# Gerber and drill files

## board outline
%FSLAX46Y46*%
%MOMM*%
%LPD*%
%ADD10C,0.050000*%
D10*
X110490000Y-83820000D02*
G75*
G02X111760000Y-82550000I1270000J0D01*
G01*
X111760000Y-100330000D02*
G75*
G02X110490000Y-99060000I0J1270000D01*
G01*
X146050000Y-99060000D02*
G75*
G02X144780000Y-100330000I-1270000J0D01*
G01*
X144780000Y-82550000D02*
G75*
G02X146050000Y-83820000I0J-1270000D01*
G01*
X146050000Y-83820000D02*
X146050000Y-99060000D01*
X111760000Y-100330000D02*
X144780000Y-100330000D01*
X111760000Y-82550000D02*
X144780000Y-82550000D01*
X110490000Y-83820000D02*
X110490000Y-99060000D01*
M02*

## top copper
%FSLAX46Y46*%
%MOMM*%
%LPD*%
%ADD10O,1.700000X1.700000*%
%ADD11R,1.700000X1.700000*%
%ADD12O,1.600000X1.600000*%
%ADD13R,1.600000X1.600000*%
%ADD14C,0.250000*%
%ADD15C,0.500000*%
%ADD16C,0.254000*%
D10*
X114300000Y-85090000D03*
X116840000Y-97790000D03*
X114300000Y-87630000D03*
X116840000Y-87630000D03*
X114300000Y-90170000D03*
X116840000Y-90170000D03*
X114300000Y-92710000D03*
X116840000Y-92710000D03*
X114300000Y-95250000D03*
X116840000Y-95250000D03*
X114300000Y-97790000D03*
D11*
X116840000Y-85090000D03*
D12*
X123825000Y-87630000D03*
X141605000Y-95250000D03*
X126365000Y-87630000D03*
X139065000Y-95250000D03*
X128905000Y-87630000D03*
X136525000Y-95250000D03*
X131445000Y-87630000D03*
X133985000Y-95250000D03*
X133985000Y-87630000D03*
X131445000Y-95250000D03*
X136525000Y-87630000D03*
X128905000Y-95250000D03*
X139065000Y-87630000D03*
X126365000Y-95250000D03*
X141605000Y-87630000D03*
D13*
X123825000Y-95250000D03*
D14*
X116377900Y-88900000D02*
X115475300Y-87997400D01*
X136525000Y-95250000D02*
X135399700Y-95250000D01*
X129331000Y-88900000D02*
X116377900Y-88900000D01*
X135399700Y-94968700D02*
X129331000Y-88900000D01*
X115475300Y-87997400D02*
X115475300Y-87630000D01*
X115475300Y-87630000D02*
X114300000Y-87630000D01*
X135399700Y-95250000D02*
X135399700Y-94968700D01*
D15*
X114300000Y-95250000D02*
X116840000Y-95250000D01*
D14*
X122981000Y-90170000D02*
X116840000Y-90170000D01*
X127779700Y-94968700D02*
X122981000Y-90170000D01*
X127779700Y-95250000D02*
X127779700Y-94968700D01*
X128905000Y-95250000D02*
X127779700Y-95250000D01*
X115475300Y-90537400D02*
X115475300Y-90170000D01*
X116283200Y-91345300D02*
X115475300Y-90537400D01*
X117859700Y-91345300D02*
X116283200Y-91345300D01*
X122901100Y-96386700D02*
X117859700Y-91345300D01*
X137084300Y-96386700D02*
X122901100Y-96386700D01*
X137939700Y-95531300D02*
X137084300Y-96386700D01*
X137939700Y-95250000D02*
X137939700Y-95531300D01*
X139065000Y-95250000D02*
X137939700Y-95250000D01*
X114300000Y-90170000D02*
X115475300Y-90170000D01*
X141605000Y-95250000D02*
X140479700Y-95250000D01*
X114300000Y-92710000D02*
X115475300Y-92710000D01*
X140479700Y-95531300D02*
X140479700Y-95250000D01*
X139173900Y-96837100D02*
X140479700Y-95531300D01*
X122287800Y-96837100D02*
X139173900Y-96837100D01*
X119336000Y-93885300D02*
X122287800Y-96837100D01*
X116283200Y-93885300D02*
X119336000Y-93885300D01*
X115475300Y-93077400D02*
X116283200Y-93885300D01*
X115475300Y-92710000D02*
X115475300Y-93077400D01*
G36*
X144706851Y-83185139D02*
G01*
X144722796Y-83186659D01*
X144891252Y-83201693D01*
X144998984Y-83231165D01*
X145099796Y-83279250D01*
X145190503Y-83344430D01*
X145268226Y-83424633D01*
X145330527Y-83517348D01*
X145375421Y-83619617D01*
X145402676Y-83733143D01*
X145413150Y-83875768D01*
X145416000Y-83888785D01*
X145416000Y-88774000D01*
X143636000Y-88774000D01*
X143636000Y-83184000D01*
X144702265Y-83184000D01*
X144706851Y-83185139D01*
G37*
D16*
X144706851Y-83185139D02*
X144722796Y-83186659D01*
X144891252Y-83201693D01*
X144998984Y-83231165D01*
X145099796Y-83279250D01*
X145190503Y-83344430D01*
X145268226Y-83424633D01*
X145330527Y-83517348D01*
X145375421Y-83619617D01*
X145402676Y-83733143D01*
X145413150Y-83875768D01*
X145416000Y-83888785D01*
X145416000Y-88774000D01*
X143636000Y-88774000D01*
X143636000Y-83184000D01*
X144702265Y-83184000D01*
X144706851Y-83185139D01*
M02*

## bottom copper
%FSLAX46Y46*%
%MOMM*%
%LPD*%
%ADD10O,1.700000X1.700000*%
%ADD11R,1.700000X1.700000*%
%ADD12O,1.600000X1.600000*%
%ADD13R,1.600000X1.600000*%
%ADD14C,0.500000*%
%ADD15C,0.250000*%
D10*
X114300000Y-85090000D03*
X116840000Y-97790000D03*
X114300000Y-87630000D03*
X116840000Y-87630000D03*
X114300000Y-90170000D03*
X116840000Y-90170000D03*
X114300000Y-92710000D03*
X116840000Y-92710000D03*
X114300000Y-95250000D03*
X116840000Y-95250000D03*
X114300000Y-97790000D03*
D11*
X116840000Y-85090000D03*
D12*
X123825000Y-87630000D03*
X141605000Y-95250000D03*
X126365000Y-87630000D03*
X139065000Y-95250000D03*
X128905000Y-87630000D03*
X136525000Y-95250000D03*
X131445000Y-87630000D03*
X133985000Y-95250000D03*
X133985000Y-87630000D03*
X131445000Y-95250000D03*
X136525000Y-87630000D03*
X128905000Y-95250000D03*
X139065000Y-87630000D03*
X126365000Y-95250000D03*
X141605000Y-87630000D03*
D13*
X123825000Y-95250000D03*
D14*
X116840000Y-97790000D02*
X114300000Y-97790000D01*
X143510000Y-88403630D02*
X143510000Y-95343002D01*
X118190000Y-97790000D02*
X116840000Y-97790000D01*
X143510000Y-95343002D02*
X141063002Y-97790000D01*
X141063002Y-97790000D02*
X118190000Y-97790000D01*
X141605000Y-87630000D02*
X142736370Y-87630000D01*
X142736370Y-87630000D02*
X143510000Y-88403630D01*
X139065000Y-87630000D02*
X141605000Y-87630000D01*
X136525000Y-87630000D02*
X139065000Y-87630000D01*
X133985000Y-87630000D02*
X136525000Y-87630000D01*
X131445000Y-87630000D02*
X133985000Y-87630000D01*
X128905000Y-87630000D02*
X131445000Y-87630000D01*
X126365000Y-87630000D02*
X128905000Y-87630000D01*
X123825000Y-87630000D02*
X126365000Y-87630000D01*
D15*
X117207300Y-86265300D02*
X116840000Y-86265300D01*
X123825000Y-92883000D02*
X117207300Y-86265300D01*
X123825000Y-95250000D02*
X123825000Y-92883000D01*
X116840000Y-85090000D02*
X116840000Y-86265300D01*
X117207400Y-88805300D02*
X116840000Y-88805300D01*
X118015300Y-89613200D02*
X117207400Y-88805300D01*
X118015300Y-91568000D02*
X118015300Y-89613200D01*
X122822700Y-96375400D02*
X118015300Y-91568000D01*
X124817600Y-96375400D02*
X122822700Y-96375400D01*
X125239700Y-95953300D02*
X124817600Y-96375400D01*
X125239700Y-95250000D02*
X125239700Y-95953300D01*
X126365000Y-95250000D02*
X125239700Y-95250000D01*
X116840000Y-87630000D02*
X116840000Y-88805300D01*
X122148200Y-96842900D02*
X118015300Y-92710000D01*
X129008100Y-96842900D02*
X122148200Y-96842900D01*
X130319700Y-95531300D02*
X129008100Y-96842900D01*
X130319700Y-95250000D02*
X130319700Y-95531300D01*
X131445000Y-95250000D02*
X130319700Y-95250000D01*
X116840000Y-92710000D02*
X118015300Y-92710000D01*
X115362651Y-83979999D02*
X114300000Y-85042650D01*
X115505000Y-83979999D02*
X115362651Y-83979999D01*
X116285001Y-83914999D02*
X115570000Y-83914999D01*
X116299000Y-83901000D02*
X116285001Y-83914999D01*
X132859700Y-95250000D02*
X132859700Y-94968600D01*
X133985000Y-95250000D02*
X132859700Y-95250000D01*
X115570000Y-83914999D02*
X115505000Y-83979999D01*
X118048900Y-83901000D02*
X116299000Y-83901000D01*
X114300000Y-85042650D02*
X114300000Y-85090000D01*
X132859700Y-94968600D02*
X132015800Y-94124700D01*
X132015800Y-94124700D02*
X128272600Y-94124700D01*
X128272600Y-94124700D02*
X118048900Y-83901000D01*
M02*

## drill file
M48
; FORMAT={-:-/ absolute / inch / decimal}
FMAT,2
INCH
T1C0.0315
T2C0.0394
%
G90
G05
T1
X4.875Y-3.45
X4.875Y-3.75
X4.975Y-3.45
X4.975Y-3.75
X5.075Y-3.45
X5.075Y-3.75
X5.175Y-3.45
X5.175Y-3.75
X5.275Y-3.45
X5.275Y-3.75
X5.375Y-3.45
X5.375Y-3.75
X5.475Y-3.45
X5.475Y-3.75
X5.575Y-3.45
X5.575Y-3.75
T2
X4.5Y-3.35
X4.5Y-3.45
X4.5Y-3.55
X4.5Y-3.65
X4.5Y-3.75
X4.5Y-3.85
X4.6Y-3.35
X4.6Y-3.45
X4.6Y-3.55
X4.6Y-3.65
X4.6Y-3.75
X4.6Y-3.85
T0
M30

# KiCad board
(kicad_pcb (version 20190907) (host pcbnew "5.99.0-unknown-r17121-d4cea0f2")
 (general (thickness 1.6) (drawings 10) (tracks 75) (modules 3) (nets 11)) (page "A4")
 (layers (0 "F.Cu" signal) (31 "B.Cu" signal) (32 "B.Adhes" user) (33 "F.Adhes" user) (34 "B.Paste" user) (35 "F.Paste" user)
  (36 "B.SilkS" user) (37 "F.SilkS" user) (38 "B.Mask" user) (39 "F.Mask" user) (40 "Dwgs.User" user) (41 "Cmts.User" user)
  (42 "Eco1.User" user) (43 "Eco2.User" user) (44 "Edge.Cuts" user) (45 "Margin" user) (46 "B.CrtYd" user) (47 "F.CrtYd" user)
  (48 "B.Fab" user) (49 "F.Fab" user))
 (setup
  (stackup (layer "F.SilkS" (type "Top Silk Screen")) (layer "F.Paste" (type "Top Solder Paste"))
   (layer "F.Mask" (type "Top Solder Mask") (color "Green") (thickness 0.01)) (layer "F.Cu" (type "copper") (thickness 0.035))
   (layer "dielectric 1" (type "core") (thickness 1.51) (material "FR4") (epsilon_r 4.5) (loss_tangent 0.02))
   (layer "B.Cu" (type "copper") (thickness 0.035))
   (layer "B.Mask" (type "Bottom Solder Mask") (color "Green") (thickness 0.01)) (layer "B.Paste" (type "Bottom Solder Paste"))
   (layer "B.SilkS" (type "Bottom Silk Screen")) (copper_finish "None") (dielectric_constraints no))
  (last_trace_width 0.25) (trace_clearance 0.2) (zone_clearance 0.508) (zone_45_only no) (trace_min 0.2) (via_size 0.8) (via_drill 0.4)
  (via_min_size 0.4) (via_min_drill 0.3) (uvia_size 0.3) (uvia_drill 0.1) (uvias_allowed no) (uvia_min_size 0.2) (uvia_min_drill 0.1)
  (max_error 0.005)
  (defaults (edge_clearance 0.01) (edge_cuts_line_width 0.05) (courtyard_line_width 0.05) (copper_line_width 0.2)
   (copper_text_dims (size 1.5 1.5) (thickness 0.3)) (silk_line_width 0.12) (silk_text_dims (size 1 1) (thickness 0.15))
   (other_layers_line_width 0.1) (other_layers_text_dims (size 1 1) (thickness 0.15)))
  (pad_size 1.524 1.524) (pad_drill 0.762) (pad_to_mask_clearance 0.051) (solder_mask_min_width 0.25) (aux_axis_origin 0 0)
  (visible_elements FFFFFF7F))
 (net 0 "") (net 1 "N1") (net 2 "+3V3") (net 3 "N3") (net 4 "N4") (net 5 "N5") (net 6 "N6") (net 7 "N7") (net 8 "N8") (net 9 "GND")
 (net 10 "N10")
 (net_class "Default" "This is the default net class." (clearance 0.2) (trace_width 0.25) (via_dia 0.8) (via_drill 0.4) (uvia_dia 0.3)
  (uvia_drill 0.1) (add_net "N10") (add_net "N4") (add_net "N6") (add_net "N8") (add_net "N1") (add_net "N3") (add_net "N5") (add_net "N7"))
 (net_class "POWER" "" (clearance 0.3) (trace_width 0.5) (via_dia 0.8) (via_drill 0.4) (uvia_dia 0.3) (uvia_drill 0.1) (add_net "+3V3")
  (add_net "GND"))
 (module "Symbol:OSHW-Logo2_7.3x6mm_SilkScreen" (layer "B.Cu") (at 123.444 91.44 180)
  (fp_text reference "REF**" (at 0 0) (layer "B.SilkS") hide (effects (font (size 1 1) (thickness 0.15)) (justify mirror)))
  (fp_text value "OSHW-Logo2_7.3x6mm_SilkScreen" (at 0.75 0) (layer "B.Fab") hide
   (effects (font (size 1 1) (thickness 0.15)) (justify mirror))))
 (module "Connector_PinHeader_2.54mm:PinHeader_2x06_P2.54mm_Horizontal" (layer "F.Cu") (at 116.84 97.79 180)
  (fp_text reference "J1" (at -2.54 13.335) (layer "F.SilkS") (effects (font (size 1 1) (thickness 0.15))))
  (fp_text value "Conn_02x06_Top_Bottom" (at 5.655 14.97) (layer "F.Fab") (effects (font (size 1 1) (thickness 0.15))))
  (pad "7" thru_hole oval (at 2.54 12.7 180) (size 1.7 1.7) (drill 1) (layers *.Cu *.Mask) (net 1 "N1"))
  (pad "6" thru_hole oval (at 0 0 180) (size 1.7 1.7) (drill 1) (layers *.Cu *.Mask) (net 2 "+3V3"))
  (pad "8" thru_hole oval (at 2.54 10.16 180) (size 1.7 1.7) (drill 1) (layers *.Cu *.Mask) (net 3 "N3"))
  (pad "2" thru_hole oval (at 0 10.16 180) (size 1.7 1.7) (drill 1) (layers *.Cu *.Mask) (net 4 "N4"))
  (pad "9" thru_hole oval (at 2.54 7.62 180) (size 1.7 1.7) (drill 1) (layers *.Cu *.Mask) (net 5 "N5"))
  (pad "3" thru_hole oval (at 0 7.62 180) (size 1.7 1.7) (drill 1) (layers *.Cu *.Mask) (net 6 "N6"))
  (pad "10" thru_hole oval (at 2.54 5.08 180) (size 1.7 1.7) (drill 1) (layers *.Cu *.Mask) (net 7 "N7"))
  (pad "4" thru_hole oval (at 0 5.08 180) (size 1.7 1.7) (drill 1) (layers *.Cu *.Mask) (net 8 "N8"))
  (pad "11" thru_hole oval (at 2.54 2.54 180) (size 1.7 1.7) (drill 1) (layers *.Cu *.Mask) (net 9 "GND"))
  (pad "5" thru_hole oval (at 0 2.54 180) (size 1.7 1.7) (drill 1) (layers *.Cu *.Mask) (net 9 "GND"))
  (pad "12" thru_hole oval (at 2.54 0 180) (size 1.7 1.7) (drill 1) (layers *.Cu *.Mask) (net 2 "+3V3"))
  (pad "1" thru_hole rect (at 0 12.7 180) (size 1.7 1.7) (drill 1) (layers *.Cu *.Mask) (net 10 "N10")))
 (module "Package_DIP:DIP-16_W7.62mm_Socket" (layer "F.Cu") (at 123.825 95.25 90)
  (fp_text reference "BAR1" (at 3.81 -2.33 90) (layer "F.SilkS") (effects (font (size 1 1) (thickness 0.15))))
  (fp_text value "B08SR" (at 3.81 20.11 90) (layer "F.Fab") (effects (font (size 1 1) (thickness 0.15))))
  (pad "16" thru_hole oval (at 7.62 0 90) (size 1.6 1.6) (drill 0.8) (layers *.Cu *.Mask) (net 2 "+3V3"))
  (pad "8" thru_hole oval (at 0 17.78 90) (size 1.6 1.6) (drill 0.8) (layers *.Cu *.Mask) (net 7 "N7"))
  (pad "15" thru_hole oval (at 7.62 2.54 90) (size 1.6 1.6) (drill 0.8) (layers *.Cu *.Mask) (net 2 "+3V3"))
  (pad "7" thru_hole oval (at 0 15.24 90) (size 1.6 1.6) (drill 0.8) (layers *.Cu *.Mask) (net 5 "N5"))
  (pad "14" thru_hole oval (at 7.62 5.08 90) (size 1.6 1.6) (drill 0.8) (layers *.Cu *.Mask) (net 2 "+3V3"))
  (pad "6" thru_hole oval (at 0 12.7 90) (size 1.6 1.6) (drill 0.8) (layers *.Cu *.Mask) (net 3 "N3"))
  (pad "13" thru_hole oval (at 7.62 7.62 90) (size 1.6 1.6) (drill 0.8) (layers *.Cu *.Mask) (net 2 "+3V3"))
  (pad "5" thru_hole oval (at 0 10.16 90) (size 1.6 1.6) (drill 0.8) (layers *.Cu *.Mask) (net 1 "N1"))
  (pad "12" thru_hole oval (at 7.62 10.16 90) (size 1.6 1.6) (drill 0.8) (layers *.Cu *.Mask) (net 2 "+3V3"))
  (pad "4" thru_hole oval (at 0 7.62 90) (size 1.6 1.6) (drill 0.8) (layers *.Cu *.Mask) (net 8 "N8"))
  (pad "11" thru_hole oval (at 7.62 12.7 90) (size 1.6 1.6) (drill 0.8) (layers *.Cu *.Mask) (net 2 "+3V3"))
  (pad "3" thru_hole oval (at 0 5.08 90) (size 1.6 1.6) (drill 0.8) (layers *.Cu *.Mask) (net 6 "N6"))
  (pad "10" thru_hole oval (at 7.62 15.24 90) (size 1.6 1.6) (drill 0.8) (layers *.Cu *.Mask) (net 2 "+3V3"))
  (pad "2" thru_hole oval (at 0 2.54 90) (size 1.6 1.6) (drill 0.8) (layers *.Cu *.Mask) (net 4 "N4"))
  (pad "9" thru_hole oval (at 7.62 17.78 90) (size 1.6 1.6) (drill 0.8) (layers *.Cu *.Mask) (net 2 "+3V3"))
  (pad "1" thru_hole rect (at 0 0 90) (size 1.6 1.6) (drill 0.8) (layers *.Cu *.Mask) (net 10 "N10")))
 (gr_arc (start 111.76 83.82) (end 111.76 82.55) (angle -90) (layer "Edge.Cuts") (width 0.05))
 (gr_arc (start 111.76 99.06) (end 110.49 99.06) (angle -90) (layer "Edge.Cuts") (width 0.05))
 (gr_arc (start 144.78 99.06) (end 144.78 100.33) (angle -90) (layer "Edge.Cuts") (width 0.05))
 (gr_arc (start 144.78 83.82) (end 146.05 83.82) (angle -90) (layer "Edge.Cuts") (width 0.05))
 (gr_line (start 146.05 83.82) (end 146.05 99.06) (layer "Edge.Cuts") (width 0.05))
 (gr_line (start 111.76 100.33) (end 144.78 100.33) (layer "Edge.Cuts") (width 0.05))
 (gr_line (start 111.76 82.55) (end 144.78 82.55) (layer "Edge.Cuts") (width 0.05))
 (gr_line (start 110.49 83.82) (end 110.49 99.06) (layer "Edge.Cuts") (width 0.05))
 (segment (start 116.3779 88.9) (end 115.4753 87.9974) (width 0.25) (layer "F.Cu") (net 3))
 (segment (start 136.525 95.25) (end 135.3997 95.25) (width 0.25) (layer "F.Cu") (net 3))
 (segment (start 129.331 88.9) (end 116.3779 88.9) (width 0.25) (layer "F.Cu") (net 3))
 (segment (start 135.3997 94.9687) (end 129.331 88.9) (width 0.25) (layer "F.Cu") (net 3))
 (segment (start 115.4753 87.9974) (end 115.4753 87.63) (width 0.25) (layer "F.Cu") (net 3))
 (segment (start 115.4753 87.63) (end 114.3 87.63) (width 0.25) (layer "F.Cu") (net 3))
 (segment (start 135.3997 95.25) (end 135.3997 94.9687) (width 0.25) (layer "F.Cu") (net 3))
 (segment (start 114.3 95.25) (end 116.84 95.25) (width 0.5) (layer "F.Cu") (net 9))
 (segment (start 116.84 97.79) (end 114.3 97.79) (width 0.5) (layer "B.Cu") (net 2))
 (segment (start 143.51 88.40363) (end 143.51 95.343002) (width 0.5) (layer "B.Cu") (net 2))
 (segment (start 118.19 97.79) (end 116.84 97.79) (width 0.5) (layer "B.Cu") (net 2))
 (segment (start 143.51 95.343002) (end 141.063002 97.79) (width 0.5) (layer "B.Cu") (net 2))
 (segment (start 141.063002 97.79) (end 118.19 97.79) (width 0.5) (layer "B.Cu") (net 2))
 (segment (start 141.605 87.63) (end 142.73637 87.63) (width 0.5) (layer "B.Cu") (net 2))
 (segment (start 142.73637 87.63) (end 143.51 88.40363) (width 0.5) (layer "B.Cu") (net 2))
 (segment (start 139.065 87.63) (end 141.605 87.63) (width 0.5) (layer "B.Cu") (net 2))
 (segment (start 136.525 87.63) (end 139.065 87.63) (width 0.5) (layer "B.Cu") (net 2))
 (segment (start 133.985 87.63) (end 136.525 87.63) (width 0.5) (layer "B.Cu") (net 2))
 (segment (start 131.445 87.63) (end 133.985 87.63) (width 0.5) (layer "B.Cu") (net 2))
 (segment (start 128.905 87.63) (end 131.445 87.63) (width 0.5) (layer "B.Cu") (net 2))
 (segment (start 126.365 87.63) (end 128.905 87.63) (width 0.5) (layer "B.Cu") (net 2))
 (segment (start 123.825 87.63) (end 126.365 87.63) (width 0.5) (layer "B.Cu") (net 2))
 (segment (start 117.2073 86.2653) (end 116.84 86.2653) (width 0.25) (layer "B.Cu") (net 10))
 (segment (start 123.825 92.883) (end 117.2073 86.2653) (width 0.25) (layer "B.Cu") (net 10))
 (segment (start 123.825 95.25) (end 123.825 92.883) (width 0.25) (layer "B.Cu") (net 10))
 (segment (start 116.84 85.09) (end 116.84 86.2653) (width 0.25) (layer "B.Cu") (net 10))
 (segment (start 117.2074 88.8053) (end 116.84 88.8053) (width 0.25) (layer "B.Cu") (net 4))
 (segment (start 118.0153 89.6132) (end 117.2074 88.8053) (width 0.25) (layer "B.Cu") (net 4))
 (segment (start 118.0153 91.568) (end 118.0153 89.6132) (width 0.25) (layer "B.Cu") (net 4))
 (segment (start 122.8227 96.3754) (end 118.0153 91.568) (width 0.25) (layer "B.Cu") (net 4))
 (segment (start 124.8176 96.3754) (end 122.8227 96.3754) (width 0.25) (layer "B.Cu") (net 4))
 (segment (start 125.2397 95.9533) (end 124.8176 96.3754) (width 0.25) (layer "B.Cu") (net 4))
 (segment (start 125.2397 95.25) (end 125.2397 95.9533) (width 0.25) (layer "B.Cu") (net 4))
 (segment (start 126.365 95.25) (end 125.2397 95.25) (width 0.25) (layer "B.Cu") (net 4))
 (segment (start 116.84 87.63) (end 116.84 88.8053) (width 0.25) (layer "B.Cu") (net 4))
 (segment (start 122.981 90.17) (end 116.84 90.17) (width 0.25) (layer "F.Cu") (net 6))
 (segment (start 127.7797 94.9687) (end 122.981 90.17) (width 0.25) (layer "F.Cu") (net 6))
 (segment (start 127.7797 95.25) (end 127.7797 94.9687) (width 0.25) (layer "F.Cu") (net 6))
 (segment (start 128.905 95.25) (end 127.7797 95.25) (width 0.25) (layer "F.Cu") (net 6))
 (segment (start 122.1482 96.8429) (end 118.0153 92.71) (width 0.25) (layer "B.Cu") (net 8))
 (segment (start 129.0081 96.8429) (end 122.1482 96.8429) (width 0.25) (layer "B.Cu") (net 8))
 (segment (start 130.3197 95.5313) (end 129.0081 96.8429) (width 0.25) (layer "B.Cu") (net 8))
 (segment (start 130.3197 95.25) (end 130.3197 95.5313) (width 0.25) (layer "B.Cu") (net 8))
 (segment (start 131.445 95.25) (end 130.3197 95.25) (width 0.25) (layer "B.Cu") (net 8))
 (segment (start 116.84 92.71) (end 118.0153 92.71) (width 0.25) (layer "B.Cu") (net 8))
 (segment (start 115.4753 90.5374) (end 115.4753 90.17) (width 0.25) (layer "F.Cu") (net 5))
 (segment (start 116.2832 91.3453) (end 115.4753 90.5374) (width 0.25) (layer "F.Cu") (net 5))
 (segment (start 117.8597 91.3453) (end 116.2832 91.3453) (width 0.25) (layer "F.Cu") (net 5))
 (segment (start 122.9011 96.3867) (end 117.8597 91.3453) (width 0.25) (layer "F.Cu") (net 5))
 (segment (start 137.0843 96.3867) (end 122.9011 96.3867) (width 0.25) (layer "F.Cu") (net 5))
 (segment (start 137.9397 95.5313) (end 137.0843 96.3867) (width 0.25) (layer "F.Cu") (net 5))
 (segment (start 137.9397 95.25) (end 137.9397 95.5313) (width 0.25) (layer "F.Cu") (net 5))
 (segment (start 139.065 95.25) (end 137.9397 95.25) (width 0.25) (layer "F.Cu") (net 5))
 (segment (start 114.3 90.17) (end 115.4753 90.17) (width 0.25) (layer "F.Cu") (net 5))
 (segment (start 141.605 95.25) (end 140.4797 95.25) (width 0.25) (layer "F.Cu") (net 7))
 (segment (start 114.3 92.71) (end 115.4753 92.71) (width 0.25) (layer "F.Cu") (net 7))
 (segment (start 140.4797 95.5313) (end 140.4797 95.25) (width 0.25) (layer "F.Cu") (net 7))
 (segment (start 139.1739 96.8371) (end 140.4797 95.5313) (width 0.25) (layer "F.Cu") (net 7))
 (segment (start 122.2878 96.8371) (end 139.1739 96.8371) (width 0.25) (layer "F.Cu") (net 7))
 (segment (start 119.336 93.8853) (end 122.2878 96.8371) (width 0.25) (layer "F.Cu") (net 7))
 (segment (start 116.2832 93.8853) (end 119.336 93.8853) (width 0.25) (layer "F.Cu") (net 7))
 (segment (start 115.4753 93.0774) (end 116.2832 93.8853) (width 0.25) (layer "F.Cu") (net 7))
 (segment (start 115.4753 92.71) (end 115.4753 93.0774) (width 0.25) (layer "F.Cu") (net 7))
 (segment (start 115.362651 83.979999) (end 114.3 85.04265) (width 0.25) (layer "B.Cu") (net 1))
 (segment (start 115.505 83.979999) (end 115.362651 83.979999) (width 0.25) (layer "B.Cu") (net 1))
 (segment (start 116.285001 83.914999) (end 115.57 83.914999) (width 0.25) (layer "B.Cu") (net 1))
 (segment (start 116.299 83.901) (end 116.285001 83.914999) (width 0.25) (layer "B.Cu") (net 1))
 (segment (start 132.8597 95.25) (end 132.8597 94.9686) (width 0.25) (layer "B.Cu") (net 1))
 (segment (start 133.985 95.25) (end 132.8597 95.25) (width 0.25) (layer "B.Cu") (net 1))
 (segment (start 115.57 83.914999) (end 115.505 83.979999) (width 0.25) (layer "B.Cu") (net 1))
 (segment (start 118.0489 83.901) (end 116.299 83.901) (width 0.25) (layer "B.Cu") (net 1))
 (segment (start 114.3 85.04265) (end 114.3 85.09) (width 0.25) (layer "B.Cu") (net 1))
 (segment (start 132.8597 94.9686) (end 132.0158 94.1247) (width 0.25) (layer "B.Cu") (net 1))
 (segment (start 132.0158 94.1247) (end 128.2726 94.1247) (width 0.25) (layer "B.Cu") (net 1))
 (segment (start 128.2726 94.1247) (end 118.0489 83.901) (width 0.25) (layer "B.Cu") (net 1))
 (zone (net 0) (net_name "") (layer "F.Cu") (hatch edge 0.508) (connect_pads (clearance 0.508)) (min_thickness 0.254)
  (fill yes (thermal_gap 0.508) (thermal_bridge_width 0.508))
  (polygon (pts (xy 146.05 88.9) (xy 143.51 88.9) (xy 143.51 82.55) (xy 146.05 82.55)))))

